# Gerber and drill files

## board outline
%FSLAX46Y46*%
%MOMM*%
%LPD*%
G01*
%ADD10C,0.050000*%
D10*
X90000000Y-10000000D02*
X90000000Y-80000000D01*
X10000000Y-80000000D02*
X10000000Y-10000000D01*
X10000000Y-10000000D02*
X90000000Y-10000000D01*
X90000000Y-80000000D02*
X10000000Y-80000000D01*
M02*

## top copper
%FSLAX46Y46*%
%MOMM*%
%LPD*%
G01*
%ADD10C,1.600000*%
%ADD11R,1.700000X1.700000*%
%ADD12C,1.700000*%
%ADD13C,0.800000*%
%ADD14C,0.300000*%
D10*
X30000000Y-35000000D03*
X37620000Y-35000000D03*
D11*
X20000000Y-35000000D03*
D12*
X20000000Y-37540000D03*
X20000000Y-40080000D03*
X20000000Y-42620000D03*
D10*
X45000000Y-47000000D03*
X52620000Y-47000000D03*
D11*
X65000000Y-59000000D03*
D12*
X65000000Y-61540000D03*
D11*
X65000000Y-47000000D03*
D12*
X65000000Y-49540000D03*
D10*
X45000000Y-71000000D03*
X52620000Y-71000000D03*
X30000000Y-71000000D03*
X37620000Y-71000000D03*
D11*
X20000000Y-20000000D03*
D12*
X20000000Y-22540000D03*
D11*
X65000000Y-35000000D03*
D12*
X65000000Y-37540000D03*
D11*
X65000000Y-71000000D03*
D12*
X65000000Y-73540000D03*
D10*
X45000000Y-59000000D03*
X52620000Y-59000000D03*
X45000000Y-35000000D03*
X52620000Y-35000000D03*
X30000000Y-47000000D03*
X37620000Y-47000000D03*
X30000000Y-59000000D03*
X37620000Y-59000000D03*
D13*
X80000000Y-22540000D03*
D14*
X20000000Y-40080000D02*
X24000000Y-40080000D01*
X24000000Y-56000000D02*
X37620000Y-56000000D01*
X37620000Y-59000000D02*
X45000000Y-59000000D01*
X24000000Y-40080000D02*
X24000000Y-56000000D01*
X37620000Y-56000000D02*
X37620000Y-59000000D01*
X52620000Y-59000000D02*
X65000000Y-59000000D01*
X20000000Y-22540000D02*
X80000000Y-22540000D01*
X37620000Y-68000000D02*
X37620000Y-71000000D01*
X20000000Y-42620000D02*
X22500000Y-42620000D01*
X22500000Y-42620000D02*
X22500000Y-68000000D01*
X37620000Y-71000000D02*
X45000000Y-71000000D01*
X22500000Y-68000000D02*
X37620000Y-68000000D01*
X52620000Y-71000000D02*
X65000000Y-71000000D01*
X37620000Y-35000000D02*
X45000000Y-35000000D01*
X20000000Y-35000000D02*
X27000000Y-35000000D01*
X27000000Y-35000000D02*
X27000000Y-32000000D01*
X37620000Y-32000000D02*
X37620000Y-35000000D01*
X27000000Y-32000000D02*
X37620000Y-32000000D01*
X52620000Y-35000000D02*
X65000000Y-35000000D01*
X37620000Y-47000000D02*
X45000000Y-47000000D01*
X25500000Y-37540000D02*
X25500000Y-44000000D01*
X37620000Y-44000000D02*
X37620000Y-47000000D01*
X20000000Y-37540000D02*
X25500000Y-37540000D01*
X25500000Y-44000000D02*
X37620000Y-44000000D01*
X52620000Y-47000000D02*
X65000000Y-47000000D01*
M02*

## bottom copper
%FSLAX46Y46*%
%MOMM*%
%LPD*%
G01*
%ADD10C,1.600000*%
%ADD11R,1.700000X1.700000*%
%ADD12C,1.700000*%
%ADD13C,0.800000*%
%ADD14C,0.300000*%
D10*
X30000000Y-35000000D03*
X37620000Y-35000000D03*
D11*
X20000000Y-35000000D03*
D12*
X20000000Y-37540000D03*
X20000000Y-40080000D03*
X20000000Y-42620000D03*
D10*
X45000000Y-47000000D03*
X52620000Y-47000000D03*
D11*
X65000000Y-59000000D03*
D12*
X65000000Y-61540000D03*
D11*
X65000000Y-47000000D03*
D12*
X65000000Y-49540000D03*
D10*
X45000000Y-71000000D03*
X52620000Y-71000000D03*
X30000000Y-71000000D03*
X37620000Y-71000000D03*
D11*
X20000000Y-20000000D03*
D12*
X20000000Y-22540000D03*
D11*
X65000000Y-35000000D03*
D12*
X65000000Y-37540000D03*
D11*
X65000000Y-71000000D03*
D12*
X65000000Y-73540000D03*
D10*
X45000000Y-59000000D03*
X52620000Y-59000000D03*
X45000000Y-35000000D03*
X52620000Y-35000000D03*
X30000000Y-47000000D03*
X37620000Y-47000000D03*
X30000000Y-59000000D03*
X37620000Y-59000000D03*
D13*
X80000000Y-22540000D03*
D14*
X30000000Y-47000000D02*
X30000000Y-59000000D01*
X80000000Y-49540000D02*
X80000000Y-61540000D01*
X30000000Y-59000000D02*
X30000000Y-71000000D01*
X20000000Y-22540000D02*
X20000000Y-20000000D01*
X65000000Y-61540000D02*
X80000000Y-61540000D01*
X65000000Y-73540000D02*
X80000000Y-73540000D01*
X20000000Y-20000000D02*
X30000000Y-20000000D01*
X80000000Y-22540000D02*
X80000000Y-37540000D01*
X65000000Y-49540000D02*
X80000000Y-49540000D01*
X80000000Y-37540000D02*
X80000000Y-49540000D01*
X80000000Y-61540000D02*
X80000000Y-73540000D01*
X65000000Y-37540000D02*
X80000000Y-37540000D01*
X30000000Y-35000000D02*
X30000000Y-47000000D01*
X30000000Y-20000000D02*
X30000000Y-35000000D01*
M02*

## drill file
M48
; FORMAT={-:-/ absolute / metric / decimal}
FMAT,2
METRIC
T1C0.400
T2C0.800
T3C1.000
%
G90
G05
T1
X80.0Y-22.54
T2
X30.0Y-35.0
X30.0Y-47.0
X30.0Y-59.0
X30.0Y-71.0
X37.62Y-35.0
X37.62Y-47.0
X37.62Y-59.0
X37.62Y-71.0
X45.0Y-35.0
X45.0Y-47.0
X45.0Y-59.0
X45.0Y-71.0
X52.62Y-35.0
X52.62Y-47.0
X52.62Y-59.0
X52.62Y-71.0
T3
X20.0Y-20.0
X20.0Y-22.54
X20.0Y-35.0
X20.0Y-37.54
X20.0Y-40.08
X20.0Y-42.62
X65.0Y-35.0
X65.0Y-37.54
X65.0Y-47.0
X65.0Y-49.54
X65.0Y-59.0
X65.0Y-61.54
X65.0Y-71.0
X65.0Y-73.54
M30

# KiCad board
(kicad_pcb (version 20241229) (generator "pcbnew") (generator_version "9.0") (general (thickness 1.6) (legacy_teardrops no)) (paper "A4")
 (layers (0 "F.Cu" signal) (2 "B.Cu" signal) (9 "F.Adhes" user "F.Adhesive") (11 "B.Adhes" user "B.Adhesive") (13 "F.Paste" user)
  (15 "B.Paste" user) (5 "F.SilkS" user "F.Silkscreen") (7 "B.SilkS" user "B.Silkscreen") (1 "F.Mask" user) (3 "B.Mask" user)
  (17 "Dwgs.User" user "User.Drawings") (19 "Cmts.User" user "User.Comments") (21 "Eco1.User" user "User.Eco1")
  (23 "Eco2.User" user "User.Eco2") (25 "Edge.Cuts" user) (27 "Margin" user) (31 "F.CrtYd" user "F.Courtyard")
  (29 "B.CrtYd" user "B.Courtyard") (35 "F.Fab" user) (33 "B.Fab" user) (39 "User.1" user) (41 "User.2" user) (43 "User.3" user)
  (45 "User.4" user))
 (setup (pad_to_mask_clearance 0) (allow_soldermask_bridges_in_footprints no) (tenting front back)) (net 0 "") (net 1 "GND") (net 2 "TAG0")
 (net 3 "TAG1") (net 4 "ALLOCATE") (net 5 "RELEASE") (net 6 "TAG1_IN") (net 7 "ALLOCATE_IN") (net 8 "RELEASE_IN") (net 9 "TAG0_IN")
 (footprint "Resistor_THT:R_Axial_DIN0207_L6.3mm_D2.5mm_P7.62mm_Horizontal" (layer "F.Cu") (at 30 35)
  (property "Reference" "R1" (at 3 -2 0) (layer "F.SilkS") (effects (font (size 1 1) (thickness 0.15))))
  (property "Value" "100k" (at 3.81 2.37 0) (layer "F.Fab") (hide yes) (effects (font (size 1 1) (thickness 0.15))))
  (pad "1" thru_hole circle (at 0 0) (size 1.6 1.6) (drill 0.8) (layers "*.Cu" "*.Mask") (remove_unused_layers no) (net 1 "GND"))
  (pad "2" thru_hole circle (at 7.62 0) (size 1.6 1.6) (drill 0.8) (layers "*.Cu" "*.Mask") (remove_unused_layers no) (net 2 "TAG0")))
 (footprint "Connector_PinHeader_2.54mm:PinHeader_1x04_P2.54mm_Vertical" (layer "F.Cu") (at 20 35)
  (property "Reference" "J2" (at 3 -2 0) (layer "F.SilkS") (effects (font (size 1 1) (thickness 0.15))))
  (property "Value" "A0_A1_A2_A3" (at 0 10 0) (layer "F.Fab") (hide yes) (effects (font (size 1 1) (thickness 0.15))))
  (pad "1" thru_hole rect (at 0 0) (size 1.7 1.7) (drill 1) (layers "*.Cu" "*.Mask") (remove_unused_layers no) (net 2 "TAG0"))
  (pad "2" thru_hole circle (at 0 2.54) (size 1.7 1.7) (drill 1) (layers "*.Cu" "*.Mask") (remove_unused_layers no) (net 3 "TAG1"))
  (pad "3" thru_hole circle (at 0 5.08) (size 1.7 1.7) (drill 1) (layers "*.Cu" "*.Mask") (remove_unused_layers no) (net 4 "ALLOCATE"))
  (pad "4" thru_hole circle (at 0 7.62) (size 1.7 1.7) (drill 1) (layers "*.Cu" "*.Mask") (remove_unused_layers no) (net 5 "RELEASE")))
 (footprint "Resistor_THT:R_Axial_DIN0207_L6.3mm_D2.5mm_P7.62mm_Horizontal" (layer "F.Cu") (at 45 47)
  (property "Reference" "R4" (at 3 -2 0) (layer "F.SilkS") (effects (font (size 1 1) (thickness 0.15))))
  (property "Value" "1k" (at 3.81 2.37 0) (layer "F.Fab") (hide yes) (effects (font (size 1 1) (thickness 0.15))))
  (pad "1" thru_hole circle (at 0 0) (size 1.6 1.6) (drill 0.8) (layers "*.Cu" "*.Mask") (remove_unused_layers no) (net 3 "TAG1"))
  (pad "2" thru_hole circle (at 7.62 0) (size 1.6 1.6) (drill 0.8) (layers "*.Cu" "*.Mask") (remove_unused_layers no) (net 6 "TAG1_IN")))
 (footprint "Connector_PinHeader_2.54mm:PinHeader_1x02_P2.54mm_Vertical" (layer "F.Cu") (at 65 59)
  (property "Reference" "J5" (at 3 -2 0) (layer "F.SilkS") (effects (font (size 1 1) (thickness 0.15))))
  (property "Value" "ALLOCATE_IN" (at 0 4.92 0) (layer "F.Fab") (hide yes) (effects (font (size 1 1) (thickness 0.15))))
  (pad "1" thru_hole rect (at 0 0) (size 1.7 1.7) (drill 1) (layers "*.Cu" "*.Mask") (remove_unused_layers no) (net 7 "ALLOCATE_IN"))
  (pad "2" thru_hole circle (at 0 2.54) (size 1.7 1.7) (drill 1) (layers "*.Cu" "*.Mask") (remove_unused_layers no) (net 1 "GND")))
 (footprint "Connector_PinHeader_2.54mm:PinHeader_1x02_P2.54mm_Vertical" (layer "F.Cu") (at 65 47)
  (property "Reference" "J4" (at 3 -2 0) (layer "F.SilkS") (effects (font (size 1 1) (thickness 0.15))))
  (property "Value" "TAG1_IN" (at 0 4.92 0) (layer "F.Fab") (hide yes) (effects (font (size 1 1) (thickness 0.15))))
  (pad "1" thru_hole rect (at 0 0) (size 1.7 1.7) (drill 1) (layers "*.Cu" "*.Mask") (remove_unused_layers no) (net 6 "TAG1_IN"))
  (pad "2" thru_hole circle (at 0 2.54) (size 1.7 1.7) (drill 1) (layers "*.Cu" "*.Mask") (remove_unused_layers no) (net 1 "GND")))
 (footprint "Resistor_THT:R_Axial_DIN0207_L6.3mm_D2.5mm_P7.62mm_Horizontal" (layer "F.Cu") (at 45 71)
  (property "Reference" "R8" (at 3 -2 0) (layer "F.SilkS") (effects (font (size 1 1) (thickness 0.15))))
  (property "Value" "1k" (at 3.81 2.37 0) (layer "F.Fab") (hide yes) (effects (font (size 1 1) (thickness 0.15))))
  (pad "1" thru_hole circle (at 0 0) (size 1.6 1.6) (drill 0.8) (layers "*.Cu" "*.Mask") (remove_unused_layers no) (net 5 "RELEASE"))
  (pad "2" thru_hole circle (at 7.62 0) (size 1.6 1.6) (drill 0.8) (layers "*.Cu" "*.Mask") (remove_unused_layers no) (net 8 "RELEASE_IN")))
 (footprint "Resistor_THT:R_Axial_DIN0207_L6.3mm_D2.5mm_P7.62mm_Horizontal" (layer "F.Cu") (at 30 71)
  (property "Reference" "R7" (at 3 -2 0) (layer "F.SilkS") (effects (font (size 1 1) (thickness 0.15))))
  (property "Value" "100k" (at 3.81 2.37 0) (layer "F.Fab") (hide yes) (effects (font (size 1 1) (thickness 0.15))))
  (pad "1" thru_hole circle (at 0 0) (size 1.6 1.6) (drill 0.8) (layers "*.Cu" "*.Mask") (remove_unused_layers no) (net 1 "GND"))
  (pad "2" thru_hole circle (at 7.62 0) (size 1.6 1.6) (drill 0.8) (layers "*.Cu" "*.Mask") (remove_unused_layers no) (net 5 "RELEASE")))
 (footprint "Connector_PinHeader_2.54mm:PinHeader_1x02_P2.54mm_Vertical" (layer "F.Cu") (at 20 20)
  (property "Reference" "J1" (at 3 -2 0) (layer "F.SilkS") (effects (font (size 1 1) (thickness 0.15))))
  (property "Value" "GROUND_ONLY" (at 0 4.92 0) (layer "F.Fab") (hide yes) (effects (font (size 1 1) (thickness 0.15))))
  (pad "1" thru_hole rect (at 0 0) (size 1.7 1.7) (drill 1) (layers "*.Cu" "*.Mask") (remove_unused_layers no) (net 1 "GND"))
  (pad "2" thru_hole circle (at 0 2.54) (size 1.7 1.7) (drill 1) (layers "*.Cu" "*.Mask") (remove_unused_layers no) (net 1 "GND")))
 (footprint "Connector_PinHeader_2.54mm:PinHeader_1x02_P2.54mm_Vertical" (layer "F.Cu") (at 65 35)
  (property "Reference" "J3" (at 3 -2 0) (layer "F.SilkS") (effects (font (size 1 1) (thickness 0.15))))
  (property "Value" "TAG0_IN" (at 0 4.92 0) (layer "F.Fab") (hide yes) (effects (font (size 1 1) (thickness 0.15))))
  (pad "1" thru_hole rect (at 0 0) (size 1.7 1.7) (drill 1) (layers "*.Cu" "*.Mask") (remove_unused_layers no) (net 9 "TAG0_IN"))
  (pad "2" thru_hole circle (at 0 2.54) (size 1.7 1.7) (drill 1) (layers "*.Cu" "*.Mask") (remove_unused_layers no) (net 1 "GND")))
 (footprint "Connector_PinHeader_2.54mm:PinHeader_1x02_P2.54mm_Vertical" (layer "F.Cu") (at 65 71)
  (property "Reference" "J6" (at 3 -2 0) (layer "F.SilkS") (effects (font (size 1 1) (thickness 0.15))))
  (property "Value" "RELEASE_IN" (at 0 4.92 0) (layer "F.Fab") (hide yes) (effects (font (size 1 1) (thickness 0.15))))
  (pad "1" thru_hole rect (at 0 0) (size 1.7 1.7) (drill 1) (layers "*.Cu" "*.Mask") (remove_unused_layers no) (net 8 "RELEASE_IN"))
  (pad "2" thru_hole circle (at 0 2.54) (size 1.7 1.7) (drill 1) (layers "*.Cu" "*.Mask") (remove_unused_layers no) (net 1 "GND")))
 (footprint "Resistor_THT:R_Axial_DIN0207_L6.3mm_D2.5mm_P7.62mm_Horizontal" (layer "F.Cu") (at 45 59)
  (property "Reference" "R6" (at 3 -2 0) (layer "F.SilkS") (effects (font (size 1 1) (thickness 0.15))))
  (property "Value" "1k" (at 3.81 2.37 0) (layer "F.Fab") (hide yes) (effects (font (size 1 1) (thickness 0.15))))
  (pad "1" thru_hole circle (at 0 0) (size 1.6 1.6) (drill 0.8) (layers "*.Cu" "*.Mask") (remove_unused_layers no) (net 4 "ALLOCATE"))
  (pad "2" thru_hole circle (at 7.62 0) (size 1.6 1.6) (drill 0.8) (layers "*.Cu" "*.Mask") (remove_unused_layers no) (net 7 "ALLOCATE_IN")))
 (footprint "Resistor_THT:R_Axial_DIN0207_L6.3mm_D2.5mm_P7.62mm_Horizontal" (layer "F.Cu") (at 45 35)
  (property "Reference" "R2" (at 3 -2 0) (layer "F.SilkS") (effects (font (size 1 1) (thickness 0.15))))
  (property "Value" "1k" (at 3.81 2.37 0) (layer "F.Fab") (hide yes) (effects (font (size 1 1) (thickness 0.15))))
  (pad "1" thru_hole circle (at 0 0) (size 1.6 1.6) (drill 0.8) (layers "*.Cu" "*.Mask") (remove_unused_layers no) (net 2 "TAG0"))
  (pad "2" thru_hole circle (at 7.62 0) (size 1.6 1.6) (drill 0.8) (layers "*.Cu" "*.Mask") (remove_unused_layers no) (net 9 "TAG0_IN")))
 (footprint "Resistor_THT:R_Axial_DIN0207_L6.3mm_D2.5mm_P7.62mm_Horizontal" (layer "F.Cu") (at 30 47)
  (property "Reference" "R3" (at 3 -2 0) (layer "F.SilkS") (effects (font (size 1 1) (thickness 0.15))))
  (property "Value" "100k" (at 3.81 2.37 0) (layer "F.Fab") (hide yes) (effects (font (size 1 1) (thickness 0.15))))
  (pad "1" thru_hole circle (at 0 0) (size 1.6 1.6) (drill 0.8) (layers "*.Cu" "*.Mask") (remove_unused_layers no) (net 1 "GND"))
  (pad "2" thru_hole circle (at 7.62 0) (size 1.6 1.6) (drill 0.8) (layers "*.Cu" "*.Mask") (remove_unused_layers no) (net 3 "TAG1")))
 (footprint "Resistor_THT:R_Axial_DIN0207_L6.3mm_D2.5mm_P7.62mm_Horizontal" (layer "F.Cu") (at 30 59)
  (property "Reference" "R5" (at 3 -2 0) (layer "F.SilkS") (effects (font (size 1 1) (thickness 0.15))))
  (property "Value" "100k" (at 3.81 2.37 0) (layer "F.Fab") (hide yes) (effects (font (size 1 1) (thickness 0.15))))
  (pad "1" thru_hole circle (at 0 0) (size 1.6 1.6) (drill 0.8) (layers "*.Cu" "*.Mask") (remove_unused_layers no) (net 1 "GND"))
  (pad "2" thru_hole circle (at 7.62 0) (size 1.6 1.6) (drill 0.8) (layers "*.Cu" "*.Mask") (remove_unused_layers no) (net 4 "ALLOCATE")))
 (gr_line (start 90 10) (end 90 80) (stroke (width 0.05) (type default)) (layer "Edge.Cuts"))
 (gr_line (start 10 80) (end 10 10) (stroke (width 0.05) (type default)) (layer "Edge.Cuts"))
 (gr_line (start 10 10) (end 90 10) (stroke (width 0.05) (type default)) (layer "Edge.Cuts"))
 (gr_line (start 90 80) (end 10 80) (stroke (width 0.05) (type default)) (layer "Edge.Cuts"))
 (segment (start 20 40.08) (end 24 40.08) (width 0.3) (layer "F.Cu") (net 4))
 (segment (start 24 56) (end 37.62 56) (width 0.3) (layer "F.Cu") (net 4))
 (segment (start 37.62 59) (end 45 59) (width 0.3) (layer "F.Cu") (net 4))
 (segment (start 24 40.08) (end 24 56) (width 0.3) (layer "F.Cu") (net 4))
 (segment (start 37.62 56) (end 37.62 59) (width 0.3) (layer "F.Cu") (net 4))
 (segment (start 52.62 59) (end 65 59) (width 0.3) (layer "F.Cu") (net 7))
 (segment (start 20 22.54) (end 80 22.54) (width 0.3) (layer "F.Cu") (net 1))
 (via (at 80 22.54) (size 0.8) (drill 0.4) (layers "F.Cu" "B.Cu") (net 1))
 (segment (start 30 47) (end 30 59) (width 0.3) (layer "B.Cu") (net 1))
 (segment (start 80 49.54) (end 80 61.54) (width 0.3) (layer "B.Cu") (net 1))
 (segment (start 30 59) (end 30 71) (width 0.3) (layer "B.Cu") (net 1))
 (segment (start 20 22.54) (end 20 20) (width 0.3) (layer "B.Cu") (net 1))
 (segment (start 65 61.54) (end 80 61.54) (width 0.3) (layer "B.Cu") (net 1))
 (segment (start 65 73.54) (end 80 73.54) (width 0.3) (layer "B.Cu") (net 1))
 (segment (start 20 20) (end 30 20) (width 0.3) (layer "B.Cu") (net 1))
 (segment (start 80 22.54) (end 80 37.54) (width 0.3) (layer "B.Cu") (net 1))
 (segment (start 65 49.54) (end 80 49.54) (width 0.3) (layer "B.Cu") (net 1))
 (segment (start 80 37.54) (end 80 49.54) (width 0.3) (layer "B.Cu") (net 1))
 (segment (start 80 61.54) (end 80 73.54) (width 0.3) (layer "B.Cu") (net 1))
 (segment (start 65 37.54) (end 80 37.54) (width 0.3) (layer "B.Cu") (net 1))
 (segment (start 30 35) (end 30 47) (width 0.3) (layer "B.Cu") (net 1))
 (segment (start 30 20) (end 30 35) (width 0.3) (layer "B.Cu") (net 1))
 (segment (start 37.62 68) (end 37.62 71) (width 0.3) (layer "F.Cu") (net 5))
 (segment (start 20 42.62) (end 22.5 42.62) (width 0.3) (layer "F.Cu") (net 5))
 (segment (start 22.5 42.62) (end 22.5 68) (width 0.3) (layer "F.Cu") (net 5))
 (segment (start 37.62 71) (end 45 71) (width 0.3) (layer "F.Cu") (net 5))
 (segment (start 22.5 68) (end 37.62 68) (width 0.3) (layer "F.Cu") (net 5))
 (segment (start 52.62 71) (end 65 71) (width 0.3) (layer "F.Cu") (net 8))
 (segment (start 37.62 35) (end 45 35) (width 0.3) (layer "F.Cu") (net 2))
 (segment (start 20 35) (end 27 35) (width 0.3) (layer "F.Cu") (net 2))
 (segment (start 27 35) (end 27 32) (width 0.3) (layer "F.Cu") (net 2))
 (segment (start 37.62 32) (end 37.62 35) (width 0.3) (layer "F.Cu") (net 2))
 (segment (start 27 32) (end 37.62 32) (width 0.3) (layer "F.Cu") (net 2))
 (segment (start 52.62 35) (end 65 35) (width 0.3) (layer "F.Cu") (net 9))
 (segment (start 37.62 47) (end 45 47) (width 0.3) (layer "F.Cu") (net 3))
 (segment (start 25.5 37.54) (end 25.5 44) (width 0.3) (layer "F.Cu") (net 3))
 (segment (start 37.62 44) (end 37.62 47) (width 0.3) (layer "F.Cu") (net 3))
 (segment (start 20 37.54) (end 25.5 37.54) (width 0.3) (layer "F.Cu") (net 3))
 (segment (start 25.5 44) (end 37.62 44) (width 0.3) (layer "F.Cu") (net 3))
 (segment (start 52.62 47) (end 65 47) (width 0.3) (layer "F.Cu") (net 6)))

